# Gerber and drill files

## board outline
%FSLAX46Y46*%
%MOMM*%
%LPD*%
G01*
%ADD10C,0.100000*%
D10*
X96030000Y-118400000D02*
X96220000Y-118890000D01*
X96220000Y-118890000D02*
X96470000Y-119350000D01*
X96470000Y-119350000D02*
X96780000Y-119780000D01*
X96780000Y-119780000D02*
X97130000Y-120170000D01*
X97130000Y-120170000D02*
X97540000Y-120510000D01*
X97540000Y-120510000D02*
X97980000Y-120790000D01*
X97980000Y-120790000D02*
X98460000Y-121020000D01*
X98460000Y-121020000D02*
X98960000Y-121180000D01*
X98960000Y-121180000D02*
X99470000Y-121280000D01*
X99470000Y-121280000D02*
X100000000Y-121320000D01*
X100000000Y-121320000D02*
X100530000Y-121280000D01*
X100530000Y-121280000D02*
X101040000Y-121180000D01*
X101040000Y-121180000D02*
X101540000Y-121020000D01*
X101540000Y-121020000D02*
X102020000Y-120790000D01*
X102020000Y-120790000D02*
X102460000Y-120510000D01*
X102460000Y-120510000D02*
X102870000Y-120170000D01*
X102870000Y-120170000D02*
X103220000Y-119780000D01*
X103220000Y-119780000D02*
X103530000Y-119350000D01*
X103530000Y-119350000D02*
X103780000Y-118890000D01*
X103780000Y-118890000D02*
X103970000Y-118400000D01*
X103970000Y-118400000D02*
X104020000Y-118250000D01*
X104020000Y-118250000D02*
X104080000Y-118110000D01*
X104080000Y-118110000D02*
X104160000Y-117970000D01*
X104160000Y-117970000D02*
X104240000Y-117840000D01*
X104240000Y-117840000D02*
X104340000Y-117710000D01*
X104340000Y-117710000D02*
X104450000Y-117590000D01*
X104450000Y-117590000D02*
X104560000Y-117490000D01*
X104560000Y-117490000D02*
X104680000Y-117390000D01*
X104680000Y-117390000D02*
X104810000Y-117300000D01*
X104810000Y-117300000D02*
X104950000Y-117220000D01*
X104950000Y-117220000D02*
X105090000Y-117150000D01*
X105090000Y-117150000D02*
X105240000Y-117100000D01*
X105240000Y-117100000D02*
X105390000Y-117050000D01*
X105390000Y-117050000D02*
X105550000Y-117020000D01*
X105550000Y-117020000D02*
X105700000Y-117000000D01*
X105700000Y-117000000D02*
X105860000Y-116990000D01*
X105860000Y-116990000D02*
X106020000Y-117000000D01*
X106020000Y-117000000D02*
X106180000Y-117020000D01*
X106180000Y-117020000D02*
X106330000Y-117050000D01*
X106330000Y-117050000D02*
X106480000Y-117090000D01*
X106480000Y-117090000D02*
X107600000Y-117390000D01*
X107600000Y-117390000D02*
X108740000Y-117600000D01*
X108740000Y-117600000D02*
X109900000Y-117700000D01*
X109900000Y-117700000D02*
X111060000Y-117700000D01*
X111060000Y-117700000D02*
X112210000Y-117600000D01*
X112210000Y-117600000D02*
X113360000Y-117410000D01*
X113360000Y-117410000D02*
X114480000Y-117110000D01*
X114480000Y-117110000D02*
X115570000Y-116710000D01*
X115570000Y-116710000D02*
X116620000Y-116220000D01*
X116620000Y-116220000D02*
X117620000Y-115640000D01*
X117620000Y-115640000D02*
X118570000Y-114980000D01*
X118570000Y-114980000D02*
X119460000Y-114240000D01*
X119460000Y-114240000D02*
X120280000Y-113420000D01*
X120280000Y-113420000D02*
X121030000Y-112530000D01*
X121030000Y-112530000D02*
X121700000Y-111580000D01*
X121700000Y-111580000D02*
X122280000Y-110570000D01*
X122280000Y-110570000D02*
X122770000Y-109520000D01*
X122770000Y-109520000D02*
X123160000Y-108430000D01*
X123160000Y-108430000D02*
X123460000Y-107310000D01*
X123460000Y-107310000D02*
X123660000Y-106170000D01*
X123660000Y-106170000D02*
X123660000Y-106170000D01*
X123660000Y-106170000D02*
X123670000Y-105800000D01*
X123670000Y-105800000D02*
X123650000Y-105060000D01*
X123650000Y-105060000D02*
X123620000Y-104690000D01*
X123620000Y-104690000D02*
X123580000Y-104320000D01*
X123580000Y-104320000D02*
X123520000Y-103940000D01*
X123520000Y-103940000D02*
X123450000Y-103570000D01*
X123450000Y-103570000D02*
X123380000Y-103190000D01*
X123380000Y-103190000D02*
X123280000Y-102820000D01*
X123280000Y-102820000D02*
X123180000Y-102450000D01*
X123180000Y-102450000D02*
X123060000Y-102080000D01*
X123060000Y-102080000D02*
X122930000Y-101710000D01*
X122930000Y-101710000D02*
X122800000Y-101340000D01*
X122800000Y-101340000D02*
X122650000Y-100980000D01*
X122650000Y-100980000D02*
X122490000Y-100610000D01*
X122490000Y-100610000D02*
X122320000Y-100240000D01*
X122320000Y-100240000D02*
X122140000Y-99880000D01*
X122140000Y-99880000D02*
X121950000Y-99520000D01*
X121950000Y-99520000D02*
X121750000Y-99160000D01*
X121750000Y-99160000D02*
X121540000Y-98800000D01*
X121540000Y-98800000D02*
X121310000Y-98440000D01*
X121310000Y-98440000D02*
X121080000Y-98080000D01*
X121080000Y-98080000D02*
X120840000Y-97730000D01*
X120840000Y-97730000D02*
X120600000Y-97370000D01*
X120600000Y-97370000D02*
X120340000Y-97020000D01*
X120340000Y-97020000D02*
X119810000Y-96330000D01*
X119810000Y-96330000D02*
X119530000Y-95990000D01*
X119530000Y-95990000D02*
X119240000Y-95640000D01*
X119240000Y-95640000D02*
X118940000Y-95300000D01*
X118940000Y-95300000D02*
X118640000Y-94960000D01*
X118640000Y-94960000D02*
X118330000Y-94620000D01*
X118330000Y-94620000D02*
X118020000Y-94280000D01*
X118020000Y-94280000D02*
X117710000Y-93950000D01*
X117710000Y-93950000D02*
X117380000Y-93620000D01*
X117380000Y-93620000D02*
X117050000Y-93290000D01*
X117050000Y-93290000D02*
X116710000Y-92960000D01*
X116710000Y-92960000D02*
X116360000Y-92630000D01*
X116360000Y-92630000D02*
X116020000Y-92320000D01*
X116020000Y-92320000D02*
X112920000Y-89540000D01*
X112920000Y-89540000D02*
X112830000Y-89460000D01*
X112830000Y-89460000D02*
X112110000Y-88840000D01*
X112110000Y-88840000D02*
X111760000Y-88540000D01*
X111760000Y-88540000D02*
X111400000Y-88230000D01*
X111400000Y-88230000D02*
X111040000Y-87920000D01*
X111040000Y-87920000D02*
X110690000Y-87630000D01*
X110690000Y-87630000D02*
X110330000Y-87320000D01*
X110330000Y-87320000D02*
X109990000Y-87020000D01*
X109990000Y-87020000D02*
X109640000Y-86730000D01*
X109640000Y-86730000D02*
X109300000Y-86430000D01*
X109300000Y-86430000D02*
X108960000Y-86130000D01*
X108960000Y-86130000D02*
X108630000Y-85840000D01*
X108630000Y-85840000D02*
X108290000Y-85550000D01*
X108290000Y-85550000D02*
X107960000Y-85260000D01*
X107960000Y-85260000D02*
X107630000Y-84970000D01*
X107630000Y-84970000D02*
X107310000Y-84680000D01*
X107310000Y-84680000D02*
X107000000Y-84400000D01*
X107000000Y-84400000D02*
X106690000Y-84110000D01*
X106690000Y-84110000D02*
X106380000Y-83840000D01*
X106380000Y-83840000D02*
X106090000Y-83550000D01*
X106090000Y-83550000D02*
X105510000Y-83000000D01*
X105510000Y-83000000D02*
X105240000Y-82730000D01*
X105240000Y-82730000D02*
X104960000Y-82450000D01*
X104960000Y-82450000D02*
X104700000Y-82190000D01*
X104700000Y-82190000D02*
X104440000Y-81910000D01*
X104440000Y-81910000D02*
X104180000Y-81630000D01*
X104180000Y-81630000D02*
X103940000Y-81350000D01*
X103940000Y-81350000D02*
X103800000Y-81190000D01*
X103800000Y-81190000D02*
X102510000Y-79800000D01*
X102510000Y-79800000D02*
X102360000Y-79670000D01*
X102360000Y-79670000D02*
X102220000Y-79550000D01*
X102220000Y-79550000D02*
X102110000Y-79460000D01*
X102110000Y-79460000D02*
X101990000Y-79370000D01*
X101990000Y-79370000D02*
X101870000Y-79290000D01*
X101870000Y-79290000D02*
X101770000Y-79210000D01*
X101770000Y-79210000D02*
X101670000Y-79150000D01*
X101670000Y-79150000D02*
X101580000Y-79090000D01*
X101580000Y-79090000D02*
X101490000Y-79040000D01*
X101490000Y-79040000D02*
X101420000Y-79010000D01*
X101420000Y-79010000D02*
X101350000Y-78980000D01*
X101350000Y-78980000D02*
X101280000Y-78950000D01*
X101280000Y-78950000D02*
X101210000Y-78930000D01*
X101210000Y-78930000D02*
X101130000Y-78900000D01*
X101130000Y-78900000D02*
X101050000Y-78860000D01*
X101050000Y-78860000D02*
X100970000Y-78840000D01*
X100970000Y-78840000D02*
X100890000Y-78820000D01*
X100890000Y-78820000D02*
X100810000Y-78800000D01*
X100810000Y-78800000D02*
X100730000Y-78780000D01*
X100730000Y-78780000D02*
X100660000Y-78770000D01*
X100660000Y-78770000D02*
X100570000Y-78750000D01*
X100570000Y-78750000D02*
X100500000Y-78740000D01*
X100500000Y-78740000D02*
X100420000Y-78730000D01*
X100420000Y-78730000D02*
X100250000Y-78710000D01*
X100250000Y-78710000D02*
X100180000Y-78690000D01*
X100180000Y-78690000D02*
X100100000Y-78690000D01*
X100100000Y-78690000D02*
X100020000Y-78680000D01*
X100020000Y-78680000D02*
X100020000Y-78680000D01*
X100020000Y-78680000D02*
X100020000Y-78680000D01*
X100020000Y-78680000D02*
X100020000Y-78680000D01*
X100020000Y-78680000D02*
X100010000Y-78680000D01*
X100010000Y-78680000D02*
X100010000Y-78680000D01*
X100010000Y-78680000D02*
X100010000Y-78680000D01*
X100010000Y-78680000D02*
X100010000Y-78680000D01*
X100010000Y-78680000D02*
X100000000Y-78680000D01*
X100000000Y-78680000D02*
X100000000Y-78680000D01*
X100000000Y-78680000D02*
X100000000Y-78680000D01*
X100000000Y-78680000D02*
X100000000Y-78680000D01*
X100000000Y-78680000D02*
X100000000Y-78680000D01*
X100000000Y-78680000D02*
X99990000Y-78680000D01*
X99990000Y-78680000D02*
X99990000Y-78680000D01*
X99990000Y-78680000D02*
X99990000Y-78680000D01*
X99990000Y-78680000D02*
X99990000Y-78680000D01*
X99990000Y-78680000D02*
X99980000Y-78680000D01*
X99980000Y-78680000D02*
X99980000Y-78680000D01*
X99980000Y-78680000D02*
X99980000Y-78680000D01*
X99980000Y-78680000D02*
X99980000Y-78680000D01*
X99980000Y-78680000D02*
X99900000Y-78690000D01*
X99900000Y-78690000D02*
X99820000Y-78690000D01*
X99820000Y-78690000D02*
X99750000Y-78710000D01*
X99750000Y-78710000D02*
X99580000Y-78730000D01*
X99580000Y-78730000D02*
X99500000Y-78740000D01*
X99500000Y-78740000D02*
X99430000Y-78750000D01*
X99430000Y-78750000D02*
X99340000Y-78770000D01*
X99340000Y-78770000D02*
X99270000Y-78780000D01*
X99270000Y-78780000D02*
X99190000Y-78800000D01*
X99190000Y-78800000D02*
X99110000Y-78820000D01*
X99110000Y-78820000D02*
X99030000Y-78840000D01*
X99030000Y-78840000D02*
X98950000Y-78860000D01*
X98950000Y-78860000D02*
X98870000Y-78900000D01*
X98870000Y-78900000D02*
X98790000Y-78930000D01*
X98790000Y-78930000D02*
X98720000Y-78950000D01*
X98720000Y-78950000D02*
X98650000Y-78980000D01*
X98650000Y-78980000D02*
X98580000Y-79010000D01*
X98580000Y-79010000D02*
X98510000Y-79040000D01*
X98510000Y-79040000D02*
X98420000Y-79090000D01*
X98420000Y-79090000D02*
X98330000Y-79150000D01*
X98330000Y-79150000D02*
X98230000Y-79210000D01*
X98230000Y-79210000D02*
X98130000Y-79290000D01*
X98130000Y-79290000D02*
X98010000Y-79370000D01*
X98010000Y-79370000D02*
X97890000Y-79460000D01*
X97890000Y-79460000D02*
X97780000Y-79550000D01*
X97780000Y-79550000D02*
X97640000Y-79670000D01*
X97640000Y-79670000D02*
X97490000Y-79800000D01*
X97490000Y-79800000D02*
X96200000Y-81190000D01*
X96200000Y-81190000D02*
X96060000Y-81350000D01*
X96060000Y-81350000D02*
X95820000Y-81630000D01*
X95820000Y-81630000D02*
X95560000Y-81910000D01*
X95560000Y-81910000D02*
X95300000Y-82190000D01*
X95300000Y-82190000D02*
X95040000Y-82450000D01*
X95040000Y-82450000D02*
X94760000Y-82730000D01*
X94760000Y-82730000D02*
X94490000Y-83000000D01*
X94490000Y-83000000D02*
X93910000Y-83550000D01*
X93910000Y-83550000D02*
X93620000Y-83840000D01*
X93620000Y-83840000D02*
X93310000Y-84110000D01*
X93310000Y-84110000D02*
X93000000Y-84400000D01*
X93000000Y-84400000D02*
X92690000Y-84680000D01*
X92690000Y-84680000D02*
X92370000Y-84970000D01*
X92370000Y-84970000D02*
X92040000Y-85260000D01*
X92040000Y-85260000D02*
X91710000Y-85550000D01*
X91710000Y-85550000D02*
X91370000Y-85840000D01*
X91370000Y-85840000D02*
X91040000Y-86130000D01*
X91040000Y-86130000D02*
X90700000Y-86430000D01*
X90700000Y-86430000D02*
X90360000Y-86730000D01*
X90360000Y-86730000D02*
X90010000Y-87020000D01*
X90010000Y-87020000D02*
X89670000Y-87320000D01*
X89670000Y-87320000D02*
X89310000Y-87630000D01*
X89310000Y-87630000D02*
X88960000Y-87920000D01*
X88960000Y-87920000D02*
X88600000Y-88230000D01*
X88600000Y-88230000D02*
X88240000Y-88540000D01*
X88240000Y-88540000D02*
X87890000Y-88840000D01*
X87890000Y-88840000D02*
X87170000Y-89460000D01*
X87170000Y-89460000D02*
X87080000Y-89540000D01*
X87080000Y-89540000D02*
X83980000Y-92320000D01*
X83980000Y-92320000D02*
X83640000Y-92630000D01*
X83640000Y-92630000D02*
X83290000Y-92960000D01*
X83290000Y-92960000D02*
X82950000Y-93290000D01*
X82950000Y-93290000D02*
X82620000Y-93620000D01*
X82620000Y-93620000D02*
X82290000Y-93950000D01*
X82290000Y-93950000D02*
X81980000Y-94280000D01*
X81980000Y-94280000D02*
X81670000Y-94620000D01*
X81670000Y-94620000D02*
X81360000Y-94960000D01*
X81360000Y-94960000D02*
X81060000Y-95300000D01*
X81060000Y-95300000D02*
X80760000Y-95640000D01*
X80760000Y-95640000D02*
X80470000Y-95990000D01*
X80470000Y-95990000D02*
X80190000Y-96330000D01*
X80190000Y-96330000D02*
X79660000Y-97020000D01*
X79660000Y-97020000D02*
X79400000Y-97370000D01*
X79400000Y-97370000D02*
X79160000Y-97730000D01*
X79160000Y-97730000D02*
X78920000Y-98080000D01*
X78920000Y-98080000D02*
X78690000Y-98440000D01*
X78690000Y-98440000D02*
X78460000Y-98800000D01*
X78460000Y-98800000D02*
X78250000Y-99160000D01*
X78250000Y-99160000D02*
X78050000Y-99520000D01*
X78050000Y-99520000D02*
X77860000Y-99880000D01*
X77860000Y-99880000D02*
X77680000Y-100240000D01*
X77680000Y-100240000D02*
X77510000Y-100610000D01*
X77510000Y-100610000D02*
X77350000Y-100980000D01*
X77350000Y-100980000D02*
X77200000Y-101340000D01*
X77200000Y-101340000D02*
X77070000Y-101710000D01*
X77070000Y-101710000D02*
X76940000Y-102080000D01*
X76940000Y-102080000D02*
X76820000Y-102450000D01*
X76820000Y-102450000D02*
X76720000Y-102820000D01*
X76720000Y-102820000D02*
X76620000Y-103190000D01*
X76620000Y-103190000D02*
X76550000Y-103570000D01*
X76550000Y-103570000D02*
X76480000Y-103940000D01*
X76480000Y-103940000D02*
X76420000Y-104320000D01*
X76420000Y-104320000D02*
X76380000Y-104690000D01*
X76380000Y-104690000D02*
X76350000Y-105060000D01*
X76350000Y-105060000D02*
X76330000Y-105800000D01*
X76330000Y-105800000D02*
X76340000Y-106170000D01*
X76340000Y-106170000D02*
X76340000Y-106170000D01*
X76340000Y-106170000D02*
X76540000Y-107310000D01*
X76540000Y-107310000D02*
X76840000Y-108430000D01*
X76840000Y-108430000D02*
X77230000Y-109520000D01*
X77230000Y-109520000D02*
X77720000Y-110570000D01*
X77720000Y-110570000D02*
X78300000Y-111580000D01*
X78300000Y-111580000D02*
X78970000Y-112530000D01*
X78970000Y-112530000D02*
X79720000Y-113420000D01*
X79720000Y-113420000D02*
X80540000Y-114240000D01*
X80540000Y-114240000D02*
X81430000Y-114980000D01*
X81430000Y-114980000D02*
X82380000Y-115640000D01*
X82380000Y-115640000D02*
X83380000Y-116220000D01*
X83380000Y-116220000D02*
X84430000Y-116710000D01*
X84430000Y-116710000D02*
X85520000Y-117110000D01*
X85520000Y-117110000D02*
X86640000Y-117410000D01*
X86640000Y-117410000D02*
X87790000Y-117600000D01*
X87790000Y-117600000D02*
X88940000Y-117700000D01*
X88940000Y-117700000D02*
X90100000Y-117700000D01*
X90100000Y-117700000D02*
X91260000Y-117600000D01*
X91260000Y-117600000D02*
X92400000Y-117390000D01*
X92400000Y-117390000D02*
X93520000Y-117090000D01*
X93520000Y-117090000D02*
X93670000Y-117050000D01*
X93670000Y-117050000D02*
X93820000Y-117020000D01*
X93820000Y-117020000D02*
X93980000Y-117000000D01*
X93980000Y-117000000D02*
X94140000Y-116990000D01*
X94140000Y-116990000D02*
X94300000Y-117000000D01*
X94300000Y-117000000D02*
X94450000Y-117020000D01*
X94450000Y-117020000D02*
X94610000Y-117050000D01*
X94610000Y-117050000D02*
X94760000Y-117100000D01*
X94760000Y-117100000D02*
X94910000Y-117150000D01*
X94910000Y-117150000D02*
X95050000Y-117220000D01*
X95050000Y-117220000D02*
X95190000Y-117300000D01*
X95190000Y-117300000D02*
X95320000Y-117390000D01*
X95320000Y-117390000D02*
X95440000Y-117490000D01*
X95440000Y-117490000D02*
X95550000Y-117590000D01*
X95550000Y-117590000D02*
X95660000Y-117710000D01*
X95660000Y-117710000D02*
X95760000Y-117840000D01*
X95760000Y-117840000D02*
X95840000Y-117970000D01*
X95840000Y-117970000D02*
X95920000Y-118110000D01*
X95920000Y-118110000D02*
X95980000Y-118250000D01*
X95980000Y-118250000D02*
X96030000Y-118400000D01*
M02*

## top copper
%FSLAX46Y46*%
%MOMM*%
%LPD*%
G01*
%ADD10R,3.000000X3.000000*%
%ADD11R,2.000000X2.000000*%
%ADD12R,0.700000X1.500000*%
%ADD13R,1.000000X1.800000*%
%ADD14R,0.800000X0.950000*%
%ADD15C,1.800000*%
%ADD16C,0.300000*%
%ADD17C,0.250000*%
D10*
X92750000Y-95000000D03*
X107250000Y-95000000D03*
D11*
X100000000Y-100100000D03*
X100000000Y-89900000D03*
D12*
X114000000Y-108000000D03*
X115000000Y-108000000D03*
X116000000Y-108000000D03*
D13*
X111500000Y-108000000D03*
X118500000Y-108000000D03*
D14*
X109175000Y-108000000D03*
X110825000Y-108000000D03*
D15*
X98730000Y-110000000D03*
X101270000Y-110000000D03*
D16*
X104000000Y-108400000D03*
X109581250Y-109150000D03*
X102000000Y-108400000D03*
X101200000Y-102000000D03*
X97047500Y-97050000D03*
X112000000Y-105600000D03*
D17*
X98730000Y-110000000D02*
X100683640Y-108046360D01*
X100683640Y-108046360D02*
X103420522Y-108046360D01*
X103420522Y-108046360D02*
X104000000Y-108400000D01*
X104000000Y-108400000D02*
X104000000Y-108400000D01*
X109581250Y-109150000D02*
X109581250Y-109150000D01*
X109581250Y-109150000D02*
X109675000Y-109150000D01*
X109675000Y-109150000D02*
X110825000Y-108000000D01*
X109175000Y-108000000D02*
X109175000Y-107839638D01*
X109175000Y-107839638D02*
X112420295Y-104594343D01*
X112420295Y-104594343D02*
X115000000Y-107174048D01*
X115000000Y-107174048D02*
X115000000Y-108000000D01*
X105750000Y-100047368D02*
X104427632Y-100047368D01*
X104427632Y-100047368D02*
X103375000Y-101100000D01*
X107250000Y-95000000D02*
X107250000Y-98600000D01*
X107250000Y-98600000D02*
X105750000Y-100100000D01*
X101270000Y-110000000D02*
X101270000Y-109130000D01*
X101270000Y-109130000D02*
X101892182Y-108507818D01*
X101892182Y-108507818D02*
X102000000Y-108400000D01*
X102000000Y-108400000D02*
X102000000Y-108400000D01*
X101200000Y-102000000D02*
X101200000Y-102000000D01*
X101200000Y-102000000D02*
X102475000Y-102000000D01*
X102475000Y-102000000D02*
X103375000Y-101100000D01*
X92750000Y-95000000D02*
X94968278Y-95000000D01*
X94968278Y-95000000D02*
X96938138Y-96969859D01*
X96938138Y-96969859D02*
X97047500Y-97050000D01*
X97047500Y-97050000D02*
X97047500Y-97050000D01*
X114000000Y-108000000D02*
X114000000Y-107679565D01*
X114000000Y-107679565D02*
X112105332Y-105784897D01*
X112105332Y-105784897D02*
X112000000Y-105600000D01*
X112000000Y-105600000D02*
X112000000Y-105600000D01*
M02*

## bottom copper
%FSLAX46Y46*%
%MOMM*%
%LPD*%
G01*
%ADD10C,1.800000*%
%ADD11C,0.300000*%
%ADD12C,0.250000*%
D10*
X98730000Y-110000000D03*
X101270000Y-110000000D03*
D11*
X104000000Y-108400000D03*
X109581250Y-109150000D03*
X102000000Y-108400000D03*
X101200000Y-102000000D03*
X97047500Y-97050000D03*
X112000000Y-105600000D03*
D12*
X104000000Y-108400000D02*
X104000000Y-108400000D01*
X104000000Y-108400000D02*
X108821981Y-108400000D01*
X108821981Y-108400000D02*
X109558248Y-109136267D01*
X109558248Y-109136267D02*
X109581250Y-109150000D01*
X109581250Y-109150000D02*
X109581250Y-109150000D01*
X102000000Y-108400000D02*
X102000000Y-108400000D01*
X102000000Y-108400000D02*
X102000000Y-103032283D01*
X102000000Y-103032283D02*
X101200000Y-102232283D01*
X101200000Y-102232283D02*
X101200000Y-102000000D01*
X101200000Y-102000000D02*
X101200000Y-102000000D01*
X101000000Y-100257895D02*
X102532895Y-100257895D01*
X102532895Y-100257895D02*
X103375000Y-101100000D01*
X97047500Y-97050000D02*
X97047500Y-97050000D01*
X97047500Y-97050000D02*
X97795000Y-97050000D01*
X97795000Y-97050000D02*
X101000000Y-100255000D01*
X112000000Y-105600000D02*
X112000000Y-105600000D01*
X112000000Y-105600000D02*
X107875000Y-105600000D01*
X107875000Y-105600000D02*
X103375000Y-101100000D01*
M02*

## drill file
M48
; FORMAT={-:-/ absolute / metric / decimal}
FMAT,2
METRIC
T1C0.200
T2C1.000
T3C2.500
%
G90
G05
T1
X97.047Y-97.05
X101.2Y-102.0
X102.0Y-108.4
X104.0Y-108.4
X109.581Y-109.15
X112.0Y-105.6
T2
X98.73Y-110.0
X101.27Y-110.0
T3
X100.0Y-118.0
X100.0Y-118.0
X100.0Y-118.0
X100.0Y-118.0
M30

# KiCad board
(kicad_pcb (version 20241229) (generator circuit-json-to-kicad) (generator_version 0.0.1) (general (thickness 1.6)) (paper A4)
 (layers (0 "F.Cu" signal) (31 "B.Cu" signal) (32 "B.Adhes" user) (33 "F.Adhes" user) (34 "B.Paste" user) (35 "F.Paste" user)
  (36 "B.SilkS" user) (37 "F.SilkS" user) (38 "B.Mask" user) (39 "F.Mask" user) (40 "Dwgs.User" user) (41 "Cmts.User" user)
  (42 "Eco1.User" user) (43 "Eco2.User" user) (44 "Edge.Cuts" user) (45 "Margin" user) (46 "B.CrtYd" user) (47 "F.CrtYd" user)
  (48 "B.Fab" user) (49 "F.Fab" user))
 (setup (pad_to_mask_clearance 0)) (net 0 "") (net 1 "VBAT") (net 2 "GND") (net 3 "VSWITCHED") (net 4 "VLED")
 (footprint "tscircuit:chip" (layer F.Cu) (at 100 95 0)
  (pad "1" smd rect (at -7.25 0 0) (size 3 3) (layers F.Cu F.Paste F.Mask) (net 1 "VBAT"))
  (pad "2" smd rect (at 7.25 0 0) (size 3 3) (layers F.Cu F.Paste F.Mask) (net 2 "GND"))
  (pad "3" smd rect (at 0 5.1 0) (size 2 2) (layers F.Cu F.Paste F.Mask))
  (pad "4" smd rect (at 0 -5.1 0) (size 2 2) (layers F.Cu F.Paste F.Mask))
  (pad "" np_thru_hole circle (at 0 23 0) (size 2.5 2.5) (drill 2.5) (layers *.Cu *.Mask)))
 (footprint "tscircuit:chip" (layer F.Cu) (at 115 108 0)
  (pad "1" smd rect (at -1 0 0) (size 0.7 1.5) (layers F.Cu F.Paste F.Mask) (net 1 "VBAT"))
  (pad "2" smd rect (at 0 0 0) (size 0.7 1.5) (layers F.Cu F.Paste F.Mask) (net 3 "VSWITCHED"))
  (pad "3" smd rect (at 1 0 0) (size 0.7 1.5) (layers F.Cu F.Paste F.Mask))
  (pad "4" smd rect (at -3.5 0 0) (size 1 1.8) (layers F.Cu F.Paste F.Mask))
  (pad "5" smd rect (at 3.5 0 0) (size 1 1.8) (layers F.Cu F.Paste F.Mask))
  (pad "" np_thru_hole circle (at -15 10 0) (size 2.5 2.5) (drill 2.5) (layers *.Cu *.Mask)))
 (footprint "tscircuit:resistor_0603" (layer F.Cu) (at 110 108 0)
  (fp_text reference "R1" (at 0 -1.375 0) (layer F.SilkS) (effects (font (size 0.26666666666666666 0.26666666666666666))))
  (pad "1" smd rect (at -0.8249999999999993 0 0) (size 0.8 0.95) (layers F.Cu F.Paste F.Mask) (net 3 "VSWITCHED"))
  (pad "2" smd rect (at 0.8249999999999993 0 0) (size 0.8 0.95) (layers F.Cu F.Paste F.Mask) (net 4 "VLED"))
  (pad "" np_thru_hole circle (at -10 10 0) (size 2.5 2.5) (drill 2.5) (layers *.Cu *.Mask)))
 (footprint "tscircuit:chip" (layer F.Cu) (at 100 110 0)
  (pad "1" thru_hole circle (at -1.27 0 0) (size 1.8 1.8) (drill 1) (layers *.Cu *.Mask) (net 4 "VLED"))
  (pad "2" thru_hole circle (at 1.27 0 0) (size 1.8 1.8) (drill 1) (layers *.Cu *.Mask) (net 2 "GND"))
  (pad "" np_thru_hole circle (at 0 8 0) (size 2.5 2.5) (drill 2.5) (layers *.Cu *.Mask)))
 (segment (start 98.73 110) (end 100.68364045267661 108.04635954732339) (width 0.25) (layer F.Cu) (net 4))
 (segment (start 100.68364045267661 108.04635954732339) (end 103.42052233324982 108.04635954732339) (width 0.25) (layer F.Cu) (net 4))
 (segment (start 103.42052233324982 108.04635954732339) (end 104 108.4) (width 0.25) (layer F.Cu) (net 4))
 (segment (start 104 108.4) (end 104 108.4) (width 0.25) (layer F.Cu) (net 4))
 (segment (start 104 108.4) (end 104 108.4) (width 0.25) (layer B.Cu) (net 4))
 (segment (start 104 108.4) (end 108.82198053451106 108.4) (width 0.25) (layer B.Cu) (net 4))
 (segment (start 108.82198053451106 108.4) (end 109.55824799304597 109.13626745853492) (width 0.25) (layer B.Cu) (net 4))
 (segment (start 109.55824799304597 109.13626745853492) (end 109.58125 109.15) (width 0.25) (layer B.Cu) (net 4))
 (segment (start 109.58125 109.15) (end 109.58125 109.15) (width 0.25) (layer B.Cu) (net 4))
 (segment (start 109.58125 109.15) (end 109.58125 109.15) (width 0.25) (layer F.Cu) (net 4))
 (segment (start 109.58125 109.15) (end 109.675 109.15) (width 0.25) (layer F.Cu) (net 4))
 (segment (start 109.675 109.15) (end 110.825 108) (width 0.25) (layer F.Cu) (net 4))
 (segment (start 109.175 108) (end 109.175 107.83963763059309) (width 0.25) (layer F.Cu) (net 3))
 (segment (start 109.175 107.83963763059309) (end 112.42029502771855 104.59434260287453) (width 0.25) (layer F.Cu) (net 3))
 (segment (start 112.42029502771855 104.59434260287453) (end 115 107.174047575156) (width 0.25) (layer F.Cu) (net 3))
 (segment (start 115 107.174047575156) (end 115 108) (width 0.25) (layer F.Cu) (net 3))
 (segment (start 105.75 100.04736842105262) (end 104.42763157894737 100.04736842105262) (width 0.25) (layer F.Cu) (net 2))
 (segment (start 104.42763157894737 100.04736842105262) (end 103.375 101.1) (width 0.25) (layer F.Cu) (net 2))
 (segment (start 107.25 95) (end 107.25 98.6) (width 0.25) (layer F.Cu) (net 2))
 (segment (start 107.25 98.6) (end 105.75 100.1) (width 0.25) (layer F.Cu) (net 2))
 (segment (start 101.27 110) (end 101.27 109.13) (width 0.25) (layer F.Cu) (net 2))
 (segment (start 101.27 109.13) (end 101.89218212350285 108.50781787649714) (width 0.25) (layer F.Cu) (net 2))
 (segment (start 101.89218212350285 108.50781787649714) (end 102 108.4) (width 0.25) (layer F.Cu) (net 2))
 (segment (start 102 108.4) (end 102 108.4) (width 0.25) (layer F.Cu) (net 2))
 (segment (start 102 108.4) (end 102 108.4) (width 0.25) (layer B.Cu) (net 2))
 (segment (start 102 108.4) (end 102 103.0322829033353) (width 0.25) (layer B.Cu) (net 2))
 (segment (start 102 103.0322829033353) (end 101.2 102.2322829033353) (width 0.25) (layer B.Cu) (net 2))
 (segment (start 101.2 102.2322829033353) (end 101.2 102) (width 0.25) (layer B.Cu) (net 2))
 (segment (start 101.2 102) (end 101.2 102) (width 0.25) (layer B.Cu) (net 2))
 (segment (start 101.2 102) (end 101.2 102) (width 0.25) (layer F.Cu) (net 2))
 (segment (start 101.2 102) (end 102.475 102) (width 0.25) (layer F.Cu) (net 2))
 (segment (start 102.475 102) (end 103.375 101.1) (width 0.25) (layer F.Cu) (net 2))
 (segment (start 101 100.2578947368421) (end 102.53289473684211 100.2578947368421) (width 0.25) (layer B.Cu) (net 1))
 (segment (start 102.53289473684211 100.2578947368421) (end 103.375 101.1) (width 0.25) (layer B.Cu) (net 1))
 (segment (start 92.75 95) (end 94.96827803179292 95) (width 0.25) (layer F.Cu) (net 1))
 (segment (start 94.96827803179292 95) (end 96.93813751697753 96.9698594851846) (width 0.25) (layer F.Cu) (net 1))
 (segment (start 96.93813751697753 96.9698594851846) (end 97.0475 97.05) (width 0.25) (layer F.Cu) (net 1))
 (segment (start 97.0475 97.05) (end 97.0475 97.05) (width 0.25) (layer F.Cu) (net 1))
 (segment (start 97.0475 97.05) (end 97.0475 97.05) (width 0.25) (layer B.Cu) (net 1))
 (segment (start 97.0475 97.05) (end 97.795 97.05) (width 0.25) (layer B.Cu) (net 1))
 (segment (start 97.795 97.05) (end 101 100.255) (width 0.25) (layer B.Cu) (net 1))
 (segment (start 114 108) (end 114 107.67956494164133) (width 0.25) (layer F.Cu) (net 1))
 (segment (start 114 107.67956494164133) (end 112.10533186932594 105.78489681096725) (width 0.25) (layer F.Cu) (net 1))
 (segment (start 112.10533186932594 105.78489681096725) (end 112 105.6) (width 0.25) (layer F.Cu) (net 1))
 (segment (start 112 105.6) (end 112 105.6) (width 0.25) (layer F.Cu) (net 1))
 (segment (start 112 105.6) (end 112 105.6) (width 0.25) (layer B.Cu) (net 1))
 (segment (start 112 105.6) (end 107.875 105.6) (width 0.25) (layer B.Cu) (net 1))
 (segment (start 107.875 105.6) (end 103.375 101.1) (width 0.25) (layer B.Cu) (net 1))
 (gr_line (start 96.03 118.4) (end 96.22 118.89) (width 0.1) (layer Edge.Cuts))
 (gr_line (start 96.22 118.89) (end 96.47 119.35) (width 0.1) (layer Edge.Cuts))
 (gr_line (start 96.47 119.35) (end 96.78 119.78) (width 0.1) (layer Edge.Cuts))
 (gr_line (start 96.78 119.78) (end 97.13 120.17) (width 0.1) (layer Edge.Cuts))
 (gr_line (start 97.13 120.17) (end 97.54 120.51) (width 0.1) (layer Edge.Cuts))
 (gr_line (start 97.54 120.51) (end 97.98 120.78999999999999) (width 0.1) (layer Edge.Cuts))
 (gr_line (start 97.98 120.78999999999999) (end 98.46 121.02) (width 0.1) (layer Edge.Cuts))
 (gr_line (start 98.46 121.02) (end 98.96 121.18) (width 0.1) (layer Edge.Cuts))
 (gr_line (start 98.96 121.18) (end 99.47 121.28) (width 0.1) (layer Edge.Cuts))
 (gr_line (start 99.47 121.28) (end 100 121.32) (width 0.1) (layer Edge.Cuts))
 (gr_line (start 100 121.32) (end 100.53 121.28) (width 0.1) (layer Edge.Cuts))
 (gr_line (start 100.53 121.28) (end 101.04 121.18) (width 0.1) (layer Edge.Cuts))
 (gr_line (start 101.04 121.18) (end 101.54 121.02) (width 0.1) (layer Edge.Cuts))
 (gr_line (start 101.54 121.02) (end 102.02 120.78999999999999) (width 0.1) (layer Edge.Cuts))
 (gr_line (start 102.02 120.78999999999999) (end 102.46 120.51) (width 0.1) (layer Edge.Cuts))
 (gr_line (start 102.46 120.51) (end 102.87 120.17) (width 0.1) (layer Edge.Cuts))
 (gr_line (start 102.87 120.17) (end 103.22 119.78) (width 0.1) (layer Edge.Cuts))
 (gr_line (start 103.22 119.78) (end 103.53 119.35) (width 0.1) (layer Edge.Cuts))
 (gr_line (start 103.53 119.35) (end 103.78 118.89) (width 0.1) (layer Edge.Cuts))
 (gr_line (start 103.78 118.89) (end 103.97 118.4) (width 0.1) (layer Edge.Cuts))
 (gr_line (start 103.97 118.4) (end 104.02 118.25) (width 0.1) (layer Edge.Cuts))
 (gr_line (start 104.02 118.25) (end 104.08 118.11) (width 0.1) (layer Edge.Cuts))
 (gr_line (start 104.08 118.11) (end 104.16 117.97) (width 0.1) (layer Edge.Cuts))
 (gr_line (start 104.16 117.97) (end 104.24 117.84) (width 0.1) (layer Edge.Cuts))
 (gr_line (start 104.24 117.84) (end 104.34 117.71000000000001) (width 0.1) (layer Edge.Cuts))
 (gr_line (start 104.34 117.71000000000001) (end 104.45 117.59) (width 0.1) (layer Edge.Cuts))
 (gr_line (start 104.45 117.59) (end 104.56 117.49) (width 0.1) (layer Edge.Cuts))
 (gr_line (start 104.56 117.49) (end 104.68 117.39) (width 0.1) (layer Edge.Cuts))
 (gr_line (start 104.68 117.39) (end 104.81 117.3) (width 0.1) (layer Edge.Cuts))
 (gr_line (start 104.81 117.3) (end 104.95 117.22) (width 0.1) (layer Edge.Cuts))
 (gr_line (start 104.95 117.22) (end 105.09 117.15) (width 0.1) (layer Edge.Cuts))
 (gr_line (start 105.09 117.15) (end 105.24 117.1) (width 0.1) (layer Edge.Cuts))
 (gr_line (start 105.24 117.1) (end 105.39 117.05) (width 0.1) (layer Edge.Cuts))
 (gr_line (start 105.39 117.05) (end 105.55 117.02) (width 0.1) (layer Edge.Cuts))
 (gr_line (start 105.55 117.02) (end 105.7 117) (width 0.1) (layer Edge.Cuts))
 (gr_line (start 105.7 117) (end 105.86 116.99) (width 0.1) (layer Edge.Cuts))
 (gr_line (start 105.86 116.99) (end 106.02 117) (width 0.1) (layer Edge.Cuts))
 (gr_line (start 106.02 117) (end 106.18 117.02) (width 0.1) (layer Edge.Cuts))
 (gr_line (start 106.18 117.02) (end 106.33 117.05) (width 0.1) (layer Edge.Cuts))
 (gr_line (start 106.33 117.05) (end 106.48 117.09) (width 0.1) (layer Edge.Cuts))
 (gr_line (start 106.48 117.09) (end 107.6 117.39) (width 0.1) (layer Edge.Cuts))
 (gr_line (start 107.6 117.39) (end 108.74 117.6) (width 0.1) (layer Edge.Cuts))
 (gr_line (start 108.74 117.6) (end 109.9 117.7) (width 0.1) (layer Edge.Cuts))
 (gr_line (start 109.9 117.7) (end 111.06 117.7) (width 0.1) (layer Edge.Cuts))
 (gr_line (start 111.06 117.7) (end 112.21000000000001 117.6) (width 0.1) (layer Edge.Cuts))
 (gr_line (start 112.21000000000001 117.6) (end 113.36 117.41) (width 0.1) (layer Edge.Cuts))
 (gr_line (start 113.36 117.41) (end 114.48 117.11) (width 0.1) (layer Edge.Cuts))
 (gr_line (start 114.48 117.11) (end 115.57 116.71000000000001) (width 0.1) (layer Edge.Cuts))
 (gr_line (start 115.57 116.71000000000001) (end 116.62 116.22) (width 0.1) (layer Edge.Cuts))
 (gr_line (start 116.62 116.22) (end 117.62 115.64) (width 0.1) (layer Edge.Cuts))
 (gr_line (start 117.62 115.64) (end 118.57 114.98) (width 0.1) (layer Edge.Cuts))
 (gr_line (start 118.57 114.98) (end 119.46000000000001 114.24) (width 0.1) (layer Edge.Cuts))
 (gr_line (start 119.46000000000001 114.24) (end 120.28 113.42) (width 0.1) (layer Edge.Cuts))
 (gr_line (start 120.28 113.42) (end 121.03 112.53) (width 0.1) (layer Edge.Cuts))
 (gr_line (start 121.03 112.53) (end 121.7 111.58) (width 0.1) (layer Edge.Cuts))
 (gr_line (start 121.7 111.58) (end 122.28 110.57) (width 0.1) (layer Edge.Cuts))
 (gr_line (start 122.28 110.57) (end 122.77 109.52) (width 0.1) (layer Edge.Cuts))
 (gr_line (start 122.77 109.52) (end 123.16 108.43) (width 0.1) (layer Edge.Cuts))
 (gr_line (start 123.16 108.43) (end 123.46000000000001 107.31) (width 0.1) (layer Edge.Cuts))
 (gr_line (start 123.46000000000001 107.31) (end 123.66 106.17) (width 0.1) (layer Edge.Cuts))
 (gr_line (start 123.66 106.17) (end 123.66 106.17) (width 0.1) (layer Edge.Cuts))
 (gr_line (start 123.66 106.17) (end 123.67 105.8) (width 0.1) (layer Edge.Cuts))
 (gr_line (start 123.67 105.8) (end 123.65 105.06) (width 0.1) (layer Edge.Cuts))
 (gr_line (start 123.65 105.06) (end 123.62 104.69) (width 0.1) (layer Edge.Cuts))
 (gr_line (start 123.62 104.69) (end 123.58 104.32) (width 0.1) (layer Edge.Cuts))
 (gr_line (start 123.58 104.32) (end 123.52 103.94) (width 0.1) (layer Edge.Cuts))
 (gr_line (start 123.52 103.94) (end 123.45 103.57) (width 0.1) (layer Edge.Cuts))
 (gr_line (start 123.45 103.57) (end 123.38 103.19) (width 0.1) (layer Edge.Cuts))
 (gr_line (start 123.38 103.19) (end 123.28 102.82) (width 0.1) (layer Edge.Cuts))
 (gr_line (start 123.28 102.82) (end 123.18 102.45) (width 0.1) (layer Edge.Cuts))
 (gr_line (start 123.18 102.45) (end 123.06 102.08) (width 0.1) (layer Edge.Cuts))
 (gr_line (start 123.06 102.08) (end 122.93 101.71) (width 0.1) (layer Edge.Cuts))
 (gr_line (start 122.93 101.71) (end 122.8 101.34) (width 0.1) (layer Edge.Cuts))
 (gr_line (start 122.8 101.34) (end 122.65 100.98) (width 0.1) (layer Edge.Cuts))
 (gr_line (start 122.65 100.98) (end 122.49 100.61) (width 0.1) (layer Edge.Cuts))
 (gr_line (start 122.49 100.61) (end 122.32 100.24) (width 0.1) (layer Edge.Cuts))
 (gr_line (start 122.32 100.24) (end 122.14 99.88) (width 0.1) (layer Edge.Cuts))
 (gr_line (start 122.14 99.88) (end 121.95 99.52) (width 0.1) (layer Edge.Cuts))
 (gr_line (start 121.95 99.52) (end 121.75 99.16) (width 0.1) (layer Edge.Cuts))
 (gr_line (start 121.75 99.16) (end 121.53999999999999 98.8) (width 0.1) (layer Edge.Cuts))
 (gr_line (start 121.53999999999999 98.8) (end 121.31 98.44) (width 0.1) (layer Edge.Cuts))
 (gr_line (start 121.31 98.44) (end 121.08 98.08) (width 0.1) (layer Edge.Cuts))
 (gr_line (start 121.08 98.08) (end 120.84 97.73) (width 0.1) (layer Edge.Cuts))
 (gr_line (start 120.84 97.73) (end 120.6 97.37) (width 0.1) (layer Edge.Cuts))
 (gr_line (start 120.6 97.37) (end 120.34 97.02) (width 0.1) (layer Edge.Cuts))
 (gr_line (start 120.34 97.02) (end 119.81 96.33) (width 0.1) (layer Edge.Cuts))
 (gr_line (start 119.81 96.33) (end 119.53 95.99) (width 0.1) (layer Edge.Cuts))
 (gr_line (start 119.53 95.99) (end 119.24 95.64) (width 0.1) (layer Edge.Cuts))
 (gr_line (start 119.24 95.64) (end 118.94 95.3) (width 0.1) (layer Edge.Cuts))
 (gr_line (start 118.94 95.3) (end 118.64 94.96) (width 0.1) (layer Edge.Cuts))
 (gr_line (start 118.64 94.96) (end 118.33 94.62) (width 0.1) (layer Edge.Cuts))
 (gr_line (start 118.33 94.62) (end 118.02 94.28) (width 0.1) (layer Edge.Cuts))
 (gr_line (start 118.02 94.28) (end 117.71000000000001 93.95) (width 0.1) (layer Edge.Cuts))
 (gr_line (start 117.71000000000001 93.95) (end 117.38 93.62) (width 0.1) (layer Edge.Cuts))
 (gr_line (start 117.38 93.62) (end 117.05 93.29) (width 0.1) (layer Edge.Cuts))
 (gr_line (start 117.05 93.29) (end 116.71000000000001 92.96) (width 0.1) (layer Edge.Cuts))
 (gr_line (start 116.71000000000001 92.96) (end 116.36 92.63) (width 0.1) (layer Edge.Cuts))
 (gr_line (start 116.36 92.63) (end 116.02 92.32) (width 0.1) (layer Edge.Cuts))
 (gr_line (start 116.02 92.32) (end 112.92 89.53999999999999) (width 0.1) (layer Edge.Cuts))
 (gr_line (start 112.92 89.53999999999999) (end 112.83 89.46000000000001) (width 0.1) (layer Edge.Cuts))
 (gr_line (start 112.83 89.46000000000001) (end 112.11 88.84) (width 0.1) (layer Edge.Cuts))
 (gr_line (start 112.11 88.84) (end 111.76 88.53999999999999) (width 0.1) (layer Edge.Cuts))
 (gr_line (start 111.76 88.53999999999999) (end 111.4 88.23) (width 0.1) (layer Edge.Cuts))
 (gr_line (start 111.4 88.23) (end 111.03999999999999 87.92) (width 0.1) (layer Edge.Cuts))
 (gr_line (start 111.03999999999999 87.92) (end 110.69 87.63) (width 0.1) (layer Edge.Cuts))
 (gr_line (start 110.69 87.63) (end 110.33 87.32) (width 0.1) (layer Edge.Cuts))
 (gr_line (start 110.33 87.32) (end 109.99 87.02) (width 0.1) (layer Edge.Cuts))
 (gr_line (start 109.99 87.02) (end 109.64 86.73) (width 0.1) (layer Edge.Cuts))
 (gr_line (start 109.64 86.73) (end 109.3 86.43) (width 0.1) (layer Edge.Cuts))
 (gr_line (start 109.3 86.43) (end 108.96000000000001 86.13) (width 0.1) (layer Edge.Cuts))
 (gr_line (start 108.96000000000001 86.13) (end 108.63 85.84) (width 0.1) (layer Edge.Cuts))
 (gr_line (start 108.63 85.84) (end 108.28999999999999 85.55) (width 0.1) (layer Edge.Cuts))
 (gr_line (start 108.28999999999999 85.55) (end 107.96 85.26) (width 0.1) (layer Edge.Cuts))
 (gr_line (start 107.96 85.26) (end 107.63 84.97) (width 0.1) (layer Edge.Cuts))
 (gr_line (start 107.63 84.97) (end 107.31 84.68) (width 0.1) (layer Edge.Cuts))
 (gr_line (start 107.31 84.68) (end 107 84.4) (width 0.1) (layer Edge.Cuts))
 (gr_line (start 107 84.4) (end 106.69 84.11) (width 0.1) (layer Edge.Cuts))
 (gr_line (start 106.69 84.11) (end 106.38 83.84) (width 0.1) (layer Edge.Cuts))
 (gr_line (start 106.38 83.84) (end 106.09 83.55) (width 0.1) (layer Edge.Cuts))
 (gr_line (start 106.09 83.55) (end 105.51 83) (width 0.1) (layer Edge.Cuts))
 (gr_line (start 105.51 83) (end 105.24 82.73) (width 0.1) (layer Edge.Cuts))
 (gr_line (start 105.24 82.73) (end 104.96 82.45) (width 0.1) (layer Edge.Cuts))
 (gr_line (start 104.96 82.45) (end 104.7 82.19) (width 0.1) (layer Edge.Cuts))
 (gr_line (start 104.7 82.19) (end 104.44 81.91) (width 0.1) (layer Edge.Cuts))
 (gr_line (start 104.44 81.91) (end 104.18 81.63) (width 0.1) (layer Edge.Cuts))
 (gr_line (start 104.18 81.63) (end 103.94 81.35) (width 0.1) (layer Edge.Cuts))
 (gr_line (start 103.94 81.35) (end 103.8 81.19) (width 0.1) (layer Edge.Cuts))
 (gr_line (start 103.8 81.19) (end 102.51 79.8) (width 0.1) (layer Edge.Cuts))
 (gr_line (start 102.51 79.8) (end 102.36 79.67) (width 0.1) (layer Edge.Cuts))
 (gr_line (start 102.36 79.67) (end 102.22 79.55) (width 0.1) (layer Edge.Cuts))
 (gr_line (start 102.22 79.55) (end 102.11 79.46000000000001) (width 0.1) (layer Edge.Cuts))
 (gr_line (start 102.11 79.46000000000001) (end 101.99 79.37) (width 0.1) (layer Edge.Cuts))
 (gr_line (start 101.99 79.37) (end 101.87 79.28999999999999) (width 0.1) (layer Edge.Cuts))
 (gr_line (start 101.87 79.28999999999999) (end 101.77 79.21000000000001) (width 0.1) (layer Edge.Cuts))
 (gr_line (start 101.77 79.21000000000001) (end 101.67 79.15) (width 0.1) (layer Edge.Cuts))
 (gr_line (start 101.67 79.15) (end 101.58 79.09) (width 0.1) (layer Edge.Cuts))
 (gr_line (start 101.58 79.09) (end 101.49 79.03999999999999) (width 0.1) (layer Edge.Cuts))
 (gr_line (start 101.49 79.03999999999999) (end 101.42 79.01) (width 0.1) (layer Edge.Cuts))
 (gr_line (start 101.42 79.01) (end 101.35 78.98) (width 0.1) (layer Edge.Cuts))
 (gr_line (start 101.35 78.98) (end 101.28 78.95) (width 0.1) (layer Edge.Cuts))
 (gr_line (start 101.28 78.95) (end 101.21 78.93) (width 0.1) (layer Edge.Cuts))
 (gr_line (start 101.21 78.93) (end 101.13 78.9) (width 0.1) (layer Edge.Cuts))
 (gr_line (start 101.13 78.9) (end 101.05 78.86) (width 0.1) (layer Edge.Cuts))
 (gr_line (start 101.05 78.86) (end 100.97 78.84) (width 0.1) (layer Edge.Cuts))
 (gr_line (start 100.97 78.84) (end 100.89 78.82) (width 0.1) (layer Edge.Cuts))
 (gr_line (start 100.89 78.82) (end 100.81 78.8) (width 0.1) (layer Edge.Cuts))
 (gr_line (start 100.81 78.8) (end 100.73 78.78) (width 0.1) (layer Edge.Cuts))
 (gr_line (start 100.73 78.78) (end 100.66 78.77) (width 0.1) (layer Edge.Cuts))
 (gr_line (start 100.66 78.77) (end 100.57 78.75) (width 0.1) (layer Edge.Cuts))
 (gr_line (start 100.57 78.75) (end 100.5 78.74) (width 0.1) (layer Edge.Cuts))
 (gr_line (start 100.5 78.74) (end 100.42 78.73) (width 0.1) (layer Edge.Cuts))
 (gr_line (start 100.42 78.73) (end 100.25 78.71000000000001) (width 0.1) (layer Edge.Cuts))
 (gr_line (start 100.25 78.71000000000001) (end 100.18 78.69) (width 0.1) (layer Edge.Cuts))
 (gr_line (start 100.18 78.69) (end 100.1 78.69) (width 0.1) (layer Edge.Cuts))
 (gr_line (start 100.1 78.69) (end 100.02 78.68) (width 0.1) (layer Edge.Cuts))
 (gr_line (start 100.02 78.68) (end 100.02 78.68) (width 0.1) (layer Edge.Cuts))
 (gr_line (start 100.02 78.68) (end 100.02 78.68) (width 0.1) (layer Edge.Cuts))
 (gr_line (start 100.02 78.68) (end 100.02 78.68) (width 0.1) (layer Edge.Cuts))
 (gr_line (start 100.02 78.68) (end 100.01 78.68) (width 0.1) (layer Edge.Cuts))
 (gr_line (start 100.01 78.68) (end 100.01 78.68) (width 0.1) (layer Edge.Cuts))
 (gr_line (start 100.01 78.68) (end 100.01 78.68) (width 0.1) (layer Edge.Cuts))
 (gr_line (start 100.01 78.68) (end 100.01 78.68) (width 0.1) (layer Edge.Cuts))
 (gr_line (start 100.01 78.68) (end 100 78.68) (width 0.1) (layer Edge.Cuts))
 (gr_line (start 100 78.68) (end 100 78.68) (width 0.1) (layer Edge.Cuts))
 (gr_line (start 100 78.68) (end 100 78.68) (width 0.1) (layer Edge.Cuts))
 (gr_line (start 100 78.68) (end 100 78.68) (width 0.1) (layer Edge.Cuts))
 (gr_line (start 100 78.68) (end 100 78.68) (width 0.1) (layer Edge.Cuts))
 (gr_line (start 100 78.68) (end 99.99 78.68) (width 0.1) (layer Edge.Cuts))
 (gr_line (start 99.99 78.68) (end 99.99 78.68) (width 0.1) (layer Edge.Cuts))
 (gr_line (start 99.99 78.68) (end 99.99 78.68) (width 0.1) (layer Edge.Cuts))
 (gr_line (start 99.99 78.68) (end 99.99 78.68) (width 0.1) (layer Edge.Cuts))
 (gr_line (start 99.99 78.68) (end 99.98 78.68) (width 0.1) (layer Edge.Cuts))
 (gr_line (start 99.98 78.68) (end 99.98 78.68) (width 0.1) (layer Edge.Cuts))
 (gr_line (start 99.98 78.68) (end 99.98 78.68) (width 0.1) (layer Edge.Cuts))
 (gr_line (start 99.98 78.68) (end 99.98 78.68) (width 0.1) (layer Edge.Cuts))
 (gr_line (start 99.98 78.68) (end 99.9 78.69) (width 0.1) (layer Edge.Cuts))
 (gr_line (start 99.9 78.69) (end 99.82 78.69) (width 0.1) (layer Edge.Cuts))
 (gr_line (start 99.82 78.69) (end 99.75 78.71000000000001) (width 0.1) (layer Edge.Cuts))
 (gr_line (start 99.75 78.71000000000001) (end 99.58 78.73) (width 0.1) (layer Edge.Cuts))
 (gr_line (start 99.58 78.73) (end 99.5 78.74) (width 0.1) (layer Edge.Cuts))
 (gr_line (start 99.5 78.74) (end 99.43 78.75) (width 0.1) (layer Edge.Cuts))
 (gr_line (start 99.43 78.75) (end 99.34 78.77) (width 0.1) (layer Edge.Cuts))
 (gr_line (start 99.34 78.77) (end 99.27 78.78) (width 0.1) (layer Edge.Cuts))
 (gr_line (start 99.27 78.78) (end 99.19 78.8) (width 0.1) (layer Edge.Cuts))
 (gr_line (start 99.19 78.8) (end 99.11 78.82) (width 0.1) (layer Edge.Cuts))
 (gr_line (start 99.11 78.82) (end 99.03 78.84) (width 0.1) (layer Edge.Cuts))
 (gr_line (start 99.03 78.84) (end 98.95 78.86) (width 0.1) (layer Edge.Cuts))
 (gr_line (start 98.95 78.86) (end 98.87 78.9) (width 0.1) (layer Edge.Cuts))
 (gr_line (start 98.87 78.9) (end 98.79 78.93) (width 0.1) (layer Edge.Cuts))
 (gr_line (start 98.79 78.93) (end 98.72 78.95) (width 0.1) (layer Edge.Cuts))
 (gr_line (start 98.72 78.95) (end 98.65 78.98) (width 0.1) (layer Edge.Cuts))
 (gr_line (start 98.65 78.98) (end 98.58 79.01) (width 0.1) (layer Edge.Cuts))
 (gr_line (start 98.58 79.01) (end 98.51 79.03999999999999) (width 0.1) (layer Edge.Cuts))
 (gr_line (start 98.51 79.03999999999999) (end 98.42 79.09) (width 0.1) (layer Edge.Cuts))
 (gr_line (start 98.42 79.09) (end 98.33 79.15) (width 0.1) (layer Edge.Cuts))
 (gr_line (start 98.33 79.15) (end 98.23 79.21000000000001) (width 0.1) (layer Edge.Cuts))
 (gr_line (start 98.23 79.21000000000001) (end 98.13 79.28999999999999) (width 0.1) (layer Edge.Cuts))
 (gr_line (start 98.13 79.28999999999999) (end 98.01 79.37) (width 0.1) (layer Edge.Cuts))
 (gr_line (start 98.01 79.37) (end 97.89 79.46000000000001) (width 0.1) (layer Edge.Cuts))
 (gr_line (start 97.89 79.46000000000001) (end 97.78 79.55) (width 0.1) (layer Edge.Cuts))
 (gr_line (start 97.78 79.55) (end 97.64 79.67) (width 0.1) (layer Edge.Cuts))
 (gr_line (start 97.64 79.67) (end 97.49 79.8) (width 0.1) (layer Edge.Cuts))
 (gr_line (start 97.49 79.8) (end 96.2 81.19) (width 0.1) (layer Edge.Cuts))
 (gr_line (start 96.2 81.19) (end 96.06 81.35) (width 0.1) (layer Edge.Cuts))
 (gr_line (start 96.06 81.35) (end 95.82 81.63) (width 0.1) (layer Edge.Cuts))
 (gr_line (start 95.82 81.63) (end 95.56 81.91) (width 0.1) (layer Edge.Cuts))
 (gr_line (start 95.56 81.91) (end 95.3 82.19) (width 0.1) (layer Edge.Cuts))
 (gr_line (start 95.3 82.19) (end 95.04 82.45) (width 0.1) (layer Edge.Cuts))
 (gr_line (start 95.04 82.45) (end 94.76 82.73) (width 0.1) (layer Edge.Cuts))
 (gr_line (start 94.76 82.73) (end 94.49 83) (width 0.1) (layer Edge.Cuts))
 (gr_line (start 94.49 83) (end 93.91 83.55) (width 0.1) (layer Edge.Cuts))
 (gr_line (start 93.91 83.55) (end 93.62 83.84) (width 0.1) (layer Edge.Cuts))
 (gr_line (start 93.62 83.84) (end 93.31 84.11) (width 0.1) (layer Edge.Cuts))
 (gr_line (start 93.31 84.11) (end 93 84.4) (width 0.1) (layer Edge.Cuts))
 (gr_line (start 93 84.4) (end 92.69 84.68) (width 0.1) (layer Edge.Cuts))
 (gr_line (start 92.69 84.68) (end 92.37 84.97) (width 0.1) (layer Edge.Cuts))
 (gr_line (start 92.37 84.97) (end 92.04 85.26) (width 0.1) (layer Edge.Cuts))
 (gr_line (start 92.04 85.26) (end 91.71000000000001 85.55) (width 0.1) (layer Edge.Cuts))
 (gr_line (start 91.71000000000001 85.55) (end 91.37 85.84) (width 0.1) (layer Edge.Cuts))
 (gr_line (start 91.37 85.84) (end 91.03999999999999 86.13) (width 0.1) (layer Edge.Cuts))
 (gr_line (start 91.03999999999999 86.13) (end 90.7 86.43) (width 0.1) (layer Edge.Cuts))
 (gr_line (start 90.7 86.43) (end 90.36 86.73) (width 0.1) (layer Edge.Cuts))
 (gr_line (start 90.36 86.73) (end 90.01 87.02) (width 0.1) (layer Edge.Cuts))
 (gr_line (start 90.01 87.02) (end 89.67 87.32) (width 0.1) (layer Edge.Cuts))
 (gr_line (start 89.67 87.32) (end 89.31 87.63) (width 0.1) (layer Edge.Cuts))
 (gr_line (start 89.31 87.63) (end 88.96000000000001 87.92) (width 0.1) (layer Edge.Cuts))
 (gr_line (start 88.96000000000001 87.92) (end 88.6 88.23) (width 0.1) (layer Edge.Cuts))
 (gr_line (start 88.6 88.23) (end 88.24 88.53999999999999) (width 0.1) (layer Edge.Cuts))
 (gr_line (start 88.24 88.53999999999999) (end 87.89 88.84) (width 0.1) (layer Edge.Cuts))
 (gr_line (start 87.89 88.84) (end 87.17 89.46000000000001) (width 0.1) (layer Edge.Cuts))
 (gr_line (start 87.17 89.46000000000001) (end 87.08 89.53999999999999) (width 0.1) (layer Edge.Cuts))
 (gr_line (start 87.08 89.53999999999999) (end 83.98 92.32) (width 0.1) (layer Edge.Cuts))
 (gr_line (start 83.98 92.32) (end 83.64 92.63) (width 0.1) (layer Edge.Cuts))
 (gr_line (start 83.64 92.63) (end 83.28999999999999 92.96) (width 0.1) (layer Edge.Cuts))
 (gr_line (start 83.28999999999999 92.96) (end 82.95 93.29) (width 0.1) (layer Edge.Cuts))
 (gr_line (start 82.95 93.29) (end 82.62 93.62) (width 0.1) (layer Edge.Cuts))
 (gr_line (start 82.62 93.62) (end 82.28999999999999 93.95) (width 0.1) (layer Edge.Cuts))
 (gr_line (start 82.28999999999999 93.95) (end 81.98 94.28) (width 0.1) (layer Edge.Cuts))
 (gr_line (start 81.98 94.28) (end 81.67 94.62) (width 0.1) (layer Edge.Cuts))
 (gr_line (start 81.67 94.62) (end 81.36 94.96) (width 0.1) (layer Edge.Cuts))
 (gr_line (start 81.36 94.96) (end 81.06 95.3) (width 0.1) (layer Edge.Cuts))
 (gr_line (start 81.06 95.3) (end 80.76 95.64) (width 0.1) (layer Edge.Cuts))
 (gr_line (start 80.76 95.64) (end 80.47 95.99) (width 0.1) (layer Edge.Cuts))
 (gr_line (start 80.47 95.99) (end 80.19 96.33) (width 0.1) (layer Edge.Cuts))
 (gr_line (start 80.19 96.33) (end 79.66 97.02) (width 0.1) (layer Edge.Cuts))
 (gr_line (start 79.66 97.02) (end 79.4 97.37) (width 0.1) (layer Edge.Cuts))
 (gr_line (start 79.4 97.37) (end 79.16 97.73) (width 0.1) (layer Edge.Cuts))
 (gr_line (start 79.16 97.73) (end 78.92 98.08) (width 0.1) (layer Edge.Cuts))
 (gr_line (start 78.92 98.08) (end 78.69 98.44) (width 0.1) (layer Edge.Cuts))
 (gr_line (start 78.69 98.44) (end 78.46000000000001 98.8) (width 0.1) (layer Edge.Cuts))
 (gr_line (start 78.46000000000001 98.8) (end 78.25 99.16) (width 0.1) (layer Edge.Cuts))
 (gr_line (start 78.25 99.16) (end 78.05 99.52) (width 0.1) (layer Edge.Cuts))
 (gr_line (start 78.05 99.52) (end 77.86 99.88) (width 0.1) (layer Edge.Cuts))
 (gr_line (start 77.86 99.88) (end 77.68 100.24) (width 0.1) (layer Edge.Cuts))
 (gr_line (start 77.68 100.24) (end 77.51 100.61) (width 0.1) (layer Edge.Cuts))
 (gr_line (start 77.51 100.61) (end 77.35 100.98) (width 0.1) (layer Edge.Cuts))
 (gr_line (start 77.35 100.98) (end 77.2 101.34) (width 0.1) (layer Edge.Cuts))
 (gr_line (start 77.2 101.34) (end 77.07 101.71) (width 0.1) (layer Edge.Cuts))
 (gr_line (start 77.07 101.71) (end 76.94 102.08) (width 0.1) (layer Edge.Cuts))
 (gr_line (start 76.94 102.08) (end 76.82 102.45) (width 0.1) (layer Edge.Cuts))
 (gr_line (start 76.82 102.45) (end 76.72 102.82) (width 0.1) (layer Edge.Cuts))
 (gr_line (start 76.72 102.82) (end 76.62 103.19) (width 0.1) (layer Edge.Cuts))
 (gr_line (start 76.62 103.19) (end 76.55 103.57) (width 0.1) (layer Edge.Cuts))
 (gr_line (start 76.55 103.57) (end 76.48 103.94) (width 0.1) (layer Edge.Cuts))
 (gr_line (start 76.48 103.94) (end 76.42 104.32) (width 0.1) (layer Edge.Cuts))
 (gr_line (start 76.42 104.32) (end 76.38 104.69) (width 0.1) (layer Edge.Cuts))
 (gr_line (start 76.38 104.69) (end 76.35 105.06) (width 0.1) (layer Edge.Cuts))
 (gr_line (start 76.35 105.06) (end 76.33 105.8) (width 0.1) (layer Edge.Cuts))
 (gr_line (start 76.33 105.8) (end 76.34 106.17) (width 0.1) (layer Edge.Cuts))
 (gr_line (start 76.34 106.17) (end 76.34 106.17) (width 0.1) (layer Edge.Cuts))
 (gr_line (start 76.34 106.17) (end 76.53999999999999 107.31) (width 0.1) (layer Edge.Cuts))
 (gr_line (start 76.53999999999999 107.31) (end 76.84 108.43) (width 0.1) (layer Edge.Cuts))
 (gr_line (start 76.84 108.43) (end 77.23 109.52) (width 0.1) (layer Edge.Cuts))
 (gr_line (start 77.23 109.52) (end 77.72 110.57) (width 0.1) (layer Edge.Cuts))
 (gr_line (start 77.72 110.57) (end 78.3 111.58) (width 0.1) (layer Edge.Cuts))
 (gr_line (start 78.3 111.58) (end 78.97 112.53) (width 0.1) (layer Edge.Cuts))
 (gr_line (start 78.97 112.53) (end 79.72 113.42) (width 0.1) (layer Edge.Cuts))
 (gr_line (start 79.72 113.42) (end 80.53999999999999 114.24) (width 0.1) (layer Edge.Cuts))
 (gr_line (start 80.53999999999999 114.24) (end 81.43 114.98) (width 0.1) (layer Edge.Cuts))
 (gr_line (start 81.43 114.98) (end 82.38 115.64) (width 0.1) (layer Edge.Cuts))
 (gr_line (start 82.38 115.64) (end 83.38 116.22) (width 0.1) (layer Edge.Cuts))
 (gr_line (start 83.38 116.22) (end 84.43 116.71000000000001) (width 0.1) (layer Edge.Cuts))
 (gr_line (start 84.43 116.71000000000001) (end 85.52 117.11) (width 0.1) (layer Edge.Cuts))
 (gr_line (start 85.52 117.11) (end 86.64 117.41) (width 0.1) (layer Edge.Cuts))
 (gr_line (start 86.64 117.41) (end 87.78999999999999 117.6) (width 0.1) (layer Edge.Cuts))
 (gr_line (start 87.78999999999999 117.6) (end 88.94 117.7) (width 0.1) (layer Edge.Cuts))
 (gr_line (start 88.94 117.7) (end 90.1 117.7) (width 0.1) (layer Edge.Cuts))
 (gr_line (start 90.1 117.7) (end 91.26 117.6) (width 0.1) (layer Edge.Cuts))
 (gr_line (start 91.26 117.6) (end 92.4 117.39) (width 0.1) (layer Edge.Cuts))
 (gr_line (start 92.4 117.39) (end 93.52 117.09) (width 0.1) (layer Edge.Cuts))
 (gr_line (start 93.52 117.09) (end 93.67 117.05) (width 0.1) (layer Edge.Cuts))
 (gr_line (start 93.67 117.05) (end 93.82 117.02) (width 0.1) (layer Edge.Cuts))
 (gr_line (start 93.82 117.02) (end 93.98 117) (width 0.1) (layer Edge.Cuts))
 (gr_line (start 93.98 117) (end 94.14 116.99) (width 0.1) (layer Edge.Cuts))
 (gr_line (start 94.14 116.99) (end 94.3 117) (width 0.1) (layer Edge.Cuts))
 (gr_line (start 94.3 117) (end 94.45 117.02) (width 0.1) (layer Edge.Cuts))
 (gr_line (start 94.45 117.02) (end 94.61 117.05) (width 0.1) (layer Edge.Cuts))
 (gr_line (start 94.61 117.05) (end 94.76 117.1) (width 0.1) (layer Edge.Cuts))
 (gr_line (start 94.76 117.1) (end 94.91 117.15) (width 0.1) (layer Edge.Cuts))
 (gr_line (start 94.91 117.15) (end 95.05 117.22) (width 0.1) (layer Edge.Cuts))
 (gr_line (start 95.05 117.22) (end 95.19 117.3) (width 0.1) (layer Edge.Cuts))
 (gr_line (start 95.19 117.3) (end 95.32 117.39) (width 0.1) (layer Edge.Cuts))
 (gr_line (start 95.32 117.39) (end 95.44 117.49) (width 0.1) (layer Edge.Cuts))
 (gr_line (start 95.44 117.49) (end 95.55 117.59) (width 0.1) (layer Edge.Cuts))
 (gr_line (start 95.55 117.59) (end 95.66 117.71000000000001) (width 0.1) (layer Edge.Cuts))
 (gr_line (start 95.66 117.71000000000001) (end 95.76 117.84) (width 0.1) (layer Edge.Cuts))
 (gr_line (start 95.76 117.84) (end 95.84 117.97) (width 0.1) (layer Edge.Cuts))
 (gr_line (start 95.84 117.97) (end 95.92 118.11) (width 0.1) (layer Edge.Cuts))
 (gr_line (start 95.92 118.11) (end 95.98 118.25) (width 0.1) (layer Edge.Cuts))
 (gr_line (start 95.98 118.25) (end 96.03 118.4) (width 0.1) (layer Edge.Cuts))
 (via (at 104 108.4) (size 0.3) (drill 0.2) (layers F.Cu B.Cu) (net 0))
 (via (at 109.58125 109.15) (size 0.3) (drill 0.2) (layers B.Cu F.Cu) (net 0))
 (via (at 102 108.4) (size 0.3) (drill 0.2) (layers F.Cu B.Cu) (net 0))
 (via (at 101.2 102) (size 0.3) (drill 0.2) (layers B.Cu F.Cu) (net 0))
 (via (at 97.0475 97.05) (size 0.3) (drill 0.2) (layers F.Cu B.Cu) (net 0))
 (via (at 112 105.6) (size 0.3) (drill 0.2) (layers F.Cu B.Cu) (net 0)))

